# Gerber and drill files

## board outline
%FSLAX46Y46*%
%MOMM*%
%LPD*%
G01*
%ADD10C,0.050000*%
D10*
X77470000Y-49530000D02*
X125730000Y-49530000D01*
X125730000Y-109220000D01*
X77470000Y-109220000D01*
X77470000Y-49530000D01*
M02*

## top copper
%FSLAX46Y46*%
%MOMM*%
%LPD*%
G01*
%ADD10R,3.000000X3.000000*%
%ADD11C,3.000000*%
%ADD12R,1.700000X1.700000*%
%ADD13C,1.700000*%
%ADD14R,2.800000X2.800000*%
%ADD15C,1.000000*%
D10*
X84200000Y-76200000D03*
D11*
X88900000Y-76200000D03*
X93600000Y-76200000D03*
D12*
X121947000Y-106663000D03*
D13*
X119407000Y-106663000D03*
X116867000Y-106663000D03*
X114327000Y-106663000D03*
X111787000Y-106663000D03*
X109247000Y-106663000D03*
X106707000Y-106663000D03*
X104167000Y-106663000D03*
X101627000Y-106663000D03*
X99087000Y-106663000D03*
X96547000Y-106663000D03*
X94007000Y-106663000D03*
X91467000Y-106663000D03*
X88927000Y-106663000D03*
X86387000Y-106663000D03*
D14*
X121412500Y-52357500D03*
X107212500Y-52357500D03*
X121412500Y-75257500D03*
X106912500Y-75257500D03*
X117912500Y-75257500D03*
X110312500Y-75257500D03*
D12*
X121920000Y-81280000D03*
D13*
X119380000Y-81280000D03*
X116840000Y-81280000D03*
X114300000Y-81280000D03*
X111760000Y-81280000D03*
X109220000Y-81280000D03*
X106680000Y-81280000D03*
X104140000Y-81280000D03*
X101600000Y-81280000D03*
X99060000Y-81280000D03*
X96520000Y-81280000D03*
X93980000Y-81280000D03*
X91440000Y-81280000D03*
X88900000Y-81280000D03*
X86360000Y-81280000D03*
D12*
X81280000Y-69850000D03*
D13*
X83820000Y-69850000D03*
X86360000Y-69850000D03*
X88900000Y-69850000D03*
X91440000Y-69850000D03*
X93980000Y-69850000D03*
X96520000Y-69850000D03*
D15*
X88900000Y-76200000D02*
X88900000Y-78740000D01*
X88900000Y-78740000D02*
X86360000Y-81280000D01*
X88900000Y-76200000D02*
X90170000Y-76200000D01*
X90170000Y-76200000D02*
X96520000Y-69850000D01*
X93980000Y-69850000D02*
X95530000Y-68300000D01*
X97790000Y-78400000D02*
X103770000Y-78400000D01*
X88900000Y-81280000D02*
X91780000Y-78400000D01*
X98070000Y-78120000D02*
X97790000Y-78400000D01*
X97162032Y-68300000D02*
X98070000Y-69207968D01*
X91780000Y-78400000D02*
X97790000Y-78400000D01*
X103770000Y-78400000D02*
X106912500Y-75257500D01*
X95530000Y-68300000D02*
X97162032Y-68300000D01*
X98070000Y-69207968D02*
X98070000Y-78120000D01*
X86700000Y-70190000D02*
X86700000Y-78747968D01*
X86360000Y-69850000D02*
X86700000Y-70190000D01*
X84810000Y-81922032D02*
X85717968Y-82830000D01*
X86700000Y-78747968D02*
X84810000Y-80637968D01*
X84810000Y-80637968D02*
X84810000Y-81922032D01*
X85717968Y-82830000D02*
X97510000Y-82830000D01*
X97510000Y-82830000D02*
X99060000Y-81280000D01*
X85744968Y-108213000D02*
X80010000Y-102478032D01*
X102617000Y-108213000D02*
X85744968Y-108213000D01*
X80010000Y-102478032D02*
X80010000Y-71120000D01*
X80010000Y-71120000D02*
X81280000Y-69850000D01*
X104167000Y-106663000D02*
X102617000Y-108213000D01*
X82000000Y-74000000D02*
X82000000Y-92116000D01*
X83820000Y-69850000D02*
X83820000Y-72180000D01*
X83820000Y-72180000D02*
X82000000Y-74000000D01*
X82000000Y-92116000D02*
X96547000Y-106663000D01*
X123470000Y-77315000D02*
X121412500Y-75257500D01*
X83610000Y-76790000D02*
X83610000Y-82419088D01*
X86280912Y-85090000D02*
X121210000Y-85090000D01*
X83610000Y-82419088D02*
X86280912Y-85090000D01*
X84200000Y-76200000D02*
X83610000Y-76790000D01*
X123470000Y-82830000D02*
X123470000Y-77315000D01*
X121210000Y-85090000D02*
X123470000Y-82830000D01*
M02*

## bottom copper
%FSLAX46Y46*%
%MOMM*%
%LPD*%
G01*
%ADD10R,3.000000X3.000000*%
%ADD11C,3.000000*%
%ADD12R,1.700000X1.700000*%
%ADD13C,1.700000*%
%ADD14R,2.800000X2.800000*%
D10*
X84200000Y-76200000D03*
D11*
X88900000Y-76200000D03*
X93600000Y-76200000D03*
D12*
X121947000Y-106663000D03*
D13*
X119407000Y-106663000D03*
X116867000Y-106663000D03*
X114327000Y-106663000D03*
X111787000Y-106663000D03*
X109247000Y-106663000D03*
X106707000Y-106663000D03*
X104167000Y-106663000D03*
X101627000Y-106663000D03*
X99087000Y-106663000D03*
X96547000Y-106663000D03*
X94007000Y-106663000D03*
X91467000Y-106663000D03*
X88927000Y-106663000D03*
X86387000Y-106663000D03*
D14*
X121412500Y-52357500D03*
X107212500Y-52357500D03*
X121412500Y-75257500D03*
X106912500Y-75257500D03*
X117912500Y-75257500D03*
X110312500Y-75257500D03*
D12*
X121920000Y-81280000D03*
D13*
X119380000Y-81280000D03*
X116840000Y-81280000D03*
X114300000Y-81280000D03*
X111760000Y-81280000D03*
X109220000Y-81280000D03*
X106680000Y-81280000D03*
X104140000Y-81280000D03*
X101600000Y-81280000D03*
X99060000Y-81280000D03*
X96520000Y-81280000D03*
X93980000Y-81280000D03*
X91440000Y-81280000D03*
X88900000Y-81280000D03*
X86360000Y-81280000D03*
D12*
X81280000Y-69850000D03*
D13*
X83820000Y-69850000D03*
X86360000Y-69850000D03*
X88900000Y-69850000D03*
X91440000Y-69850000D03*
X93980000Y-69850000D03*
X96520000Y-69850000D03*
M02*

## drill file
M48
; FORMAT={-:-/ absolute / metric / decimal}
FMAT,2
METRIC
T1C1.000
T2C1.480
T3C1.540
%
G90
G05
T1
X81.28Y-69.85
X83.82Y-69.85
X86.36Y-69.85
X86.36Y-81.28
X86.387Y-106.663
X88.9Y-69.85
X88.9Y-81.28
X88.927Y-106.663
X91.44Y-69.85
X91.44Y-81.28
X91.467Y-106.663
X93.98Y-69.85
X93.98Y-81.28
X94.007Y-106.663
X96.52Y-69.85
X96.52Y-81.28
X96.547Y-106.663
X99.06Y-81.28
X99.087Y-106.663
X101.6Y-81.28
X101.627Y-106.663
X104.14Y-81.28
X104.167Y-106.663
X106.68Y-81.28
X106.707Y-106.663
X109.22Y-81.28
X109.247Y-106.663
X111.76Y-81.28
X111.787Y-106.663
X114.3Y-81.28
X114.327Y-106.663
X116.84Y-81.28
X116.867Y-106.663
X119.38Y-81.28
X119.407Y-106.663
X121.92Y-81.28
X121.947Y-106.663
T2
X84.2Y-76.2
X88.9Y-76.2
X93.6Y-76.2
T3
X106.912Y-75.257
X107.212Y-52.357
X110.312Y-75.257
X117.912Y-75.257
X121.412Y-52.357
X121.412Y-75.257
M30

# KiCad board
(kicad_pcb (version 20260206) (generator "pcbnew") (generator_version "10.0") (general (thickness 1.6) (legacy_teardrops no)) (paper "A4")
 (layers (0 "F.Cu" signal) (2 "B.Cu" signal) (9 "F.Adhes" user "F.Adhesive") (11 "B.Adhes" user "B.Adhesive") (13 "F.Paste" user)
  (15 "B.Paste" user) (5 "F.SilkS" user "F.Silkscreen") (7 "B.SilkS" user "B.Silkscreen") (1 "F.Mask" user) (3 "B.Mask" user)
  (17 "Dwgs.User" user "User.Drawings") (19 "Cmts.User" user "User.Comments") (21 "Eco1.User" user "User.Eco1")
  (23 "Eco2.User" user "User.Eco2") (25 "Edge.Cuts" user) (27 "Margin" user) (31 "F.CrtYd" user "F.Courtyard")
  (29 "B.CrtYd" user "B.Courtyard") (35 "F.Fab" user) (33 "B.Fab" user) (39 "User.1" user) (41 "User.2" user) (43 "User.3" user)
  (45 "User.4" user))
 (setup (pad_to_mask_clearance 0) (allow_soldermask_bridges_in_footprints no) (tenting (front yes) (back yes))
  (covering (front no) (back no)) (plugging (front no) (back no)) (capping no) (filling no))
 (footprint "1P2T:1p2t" (layer "F.Cu") (at 88.9 76.2)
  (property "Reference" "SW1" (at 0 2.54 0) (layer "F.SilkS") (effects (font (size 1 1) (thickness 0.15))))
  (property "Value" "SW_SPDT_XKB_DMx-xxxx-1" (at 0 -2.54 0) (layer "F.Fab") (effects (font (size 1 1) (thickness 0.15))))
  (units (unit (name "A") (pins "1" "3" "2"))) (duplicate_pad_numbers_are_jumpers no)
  (pad "1" thru_hole rect (at -4.7 0) (size 3 3) (drill 1.48) (layers "*.Cu" "*.Mask") (remove_unused_layers no) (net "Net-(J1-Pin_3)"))
  (pad "2" thru_hole circle (at 0 0) (size 3 3) (drill 1.48) (layers "*.Cu" "*.Mask") (remove_unused_layers no) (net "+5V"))
  (pad "3" thru_hole circle (at 4.7 0) (size 3 3) (drill 1.48) (layers "*.Cu" "*.Mask") (remove_unused_layers no)
   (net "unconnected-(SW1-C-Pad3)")))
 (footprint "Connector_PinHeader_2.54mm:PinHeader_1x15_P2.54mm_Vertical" (layer "F.Cu") (at 121.947 106.663 -90)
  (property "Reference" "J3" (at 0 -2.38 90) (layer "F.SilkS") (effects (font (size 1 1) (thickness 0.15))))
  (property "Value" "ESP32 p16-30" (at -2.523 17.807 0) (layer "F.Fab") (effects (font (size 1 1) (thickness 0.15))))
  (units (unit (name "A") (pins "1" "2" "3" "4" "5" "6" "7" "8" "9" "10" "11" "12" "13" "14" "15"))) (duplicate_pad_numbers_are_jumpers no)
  (pad "1" thru_hole rect (at 0 0 270) (size 1.7 1.7) (drill 1) (layers "*.Cu" "*.Mask") (remove_unused_layers no)
   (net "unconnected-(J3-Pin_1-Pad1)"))
  (pad "2" thru_hole circle (at 0 2.54 270) (size 1.7 1.7) (drill 1) (layers "*.Cu" "*.Mask") (remove_unused_layers no)
   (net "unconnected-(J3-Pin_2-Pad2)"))
  (pad "3" thru_hole circle (at 0 5.08 270) (size 1.7 1.7) (drill 1) (layers "*.Cu" "*.Mask") (remove_unused_layers no)
   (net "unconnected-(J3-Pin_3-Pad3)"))
  (pad "4" thru_hole circle (at 0 7.62 270) (size 1.7 1.7) (drill 1) (layers "*.Cu" "*.Mask") (remove_unused_layers no)
   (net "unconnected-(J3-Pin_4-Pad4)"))
  (pad "5" thru_hole circle (at 0 10.16 270) (size 1.7 1.7) (drill 1) (layers "*.Cu" "*.Mask") (remove_unused_layers no)
   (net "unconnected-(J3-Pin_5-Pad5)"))
  (pad "6" thru_hole circle (at 0 12.7 270) (size 1.7 1.7) (drill 1) (layers "*.Cu" "*.Mask") (remove_unused_layers no)
   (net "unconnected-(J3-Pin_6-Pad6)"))
  (pad "7" thru_hole circle (at 0 15.24 270) (size 1.7 1.7) (drill 1) (layers "*.Cu" "*.Mask") (remove_unused_layers no)
   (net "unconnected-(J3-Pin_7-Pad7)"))
  (pad "8" thru_hole circle (at 0 17.78 270) (size 1.7 1.7) (drill 1) (layers "*.Cu" "*.Mask") (remove_unused_layers no) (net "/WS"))
  (pad "9" thru_hole circle (at 0 20.32 270) (size 1.7 1.7) (drill 1) (layers "*.Cu" "*.Mask") (remove_unused_layers no)
   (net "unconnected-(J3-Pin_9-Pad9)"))
  (pad "10" thru_hole circle (at 0 22.86 270) (size 1.7 1.7) (drill 1) (layers "*.Cu" "*.Mask") (remove_unused_layers no)
   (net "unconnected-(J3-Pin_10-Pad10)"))
  (pad "11" thru_hole circle (at 0 25.4 270) (size 1.7 1.7) (drill 1) (layers "*.Cu" "*.Mask") (remove_unused_layers no) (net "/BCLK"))
  (pad "12" thru_hole circle (at 0 27.94 270) (size 1.7 1.7) (drill 1) (layers "*.Cu" "*.Mask") (remove_unused_layers no)
   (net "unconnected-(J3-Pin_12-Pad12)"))
  (pad "13" thru_hole circle (at 0 30.48 270) (size 1.7 1.7) (drill 1) (layers "*.Cu" "*.Mask") (remove_unused_layers no)
   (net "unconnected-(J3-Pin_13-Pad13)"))
  (pad "14" thru_hole circle (at 0 33.02 270) (size 1.7 1.7) (drill 1) (layers "*.Cu" "*.Mask") (remove_unused_layers no)
   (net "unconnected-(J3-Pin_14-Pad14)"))
  (pad "15" thru_hole circle (at 0 35.56 270) (size 1.7 1.7) (drill 1) (layers "*.Cu" "*.Mask") (remove_unused_layers no)
   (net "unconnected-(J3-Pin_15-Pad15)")))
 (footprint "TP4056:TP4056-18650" (layer "F.Cu") (at 123.1125 50.6575 -90)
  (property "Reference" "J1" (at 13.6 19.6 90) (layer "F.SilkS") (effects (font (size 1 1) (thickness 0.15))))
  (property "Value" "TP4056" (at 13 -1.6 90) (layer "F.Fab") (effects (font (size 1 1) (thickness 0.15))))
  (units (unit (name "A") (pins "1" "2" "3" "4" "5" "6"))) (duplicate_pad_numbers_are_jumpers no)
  (pad "1" thru_hole rect (at 1.7 1.7 270) (size 2.8 2.8) (drill 1.54) (layers "*.Cu" "*.Mask") (remove_unused_layers no)
   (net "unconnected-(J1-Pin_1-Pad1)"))
  (pad "2" thru_hole rect (at 1.7 15.9 270) (size 2.8 2.8) (drill 1.54) (layers "*.Cu" "*.Mask") (remove_unused_layers no)
   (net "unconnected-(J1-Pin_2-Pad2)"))
  (pad "3" thru_hole rect (at 24.6 1.7 270) (size 2.8 2.8) (drill 1.54) (layers "*.Cu" "*.Mask") (remove_unused_layers no)
   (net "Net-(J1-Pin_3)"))
  (pad "4" thru_hole rect (at 24.6 16.2 270) (size 2.8 2.8) (drill 1.54) (layers "*.Cu" "*.Mask") (remove_unused_layers no) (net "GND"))
  (pad "5" thru_hole rect (at 24.6 5.2 270) (size 2.8 2.8) (drill 1.54) (layers "*.Cu" "*.Mask") (remove_unused_layers no) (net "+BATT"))
  (pad "6" thru_hole rect (at 24.6 12.8 270) (size 2.8 2.8) (drill 1.54) (layers "*.Cu" "*.Mask") (remove_unused_layers no) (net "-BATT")))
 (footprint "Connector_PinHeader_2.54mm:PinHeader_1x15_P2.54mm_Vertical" (layer "F.Cu") (at 121.92 81.28 -90)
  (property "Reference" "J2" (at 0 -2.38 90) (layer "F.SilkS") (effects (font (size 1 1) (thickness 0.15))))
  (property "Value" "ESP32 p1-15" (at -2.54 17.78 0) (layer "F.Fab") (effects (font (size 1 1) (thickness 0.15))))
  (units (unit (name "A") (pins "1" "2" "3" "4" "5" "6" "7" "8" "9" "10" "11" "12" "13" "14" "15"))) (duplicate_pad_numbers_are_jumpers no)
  (pad "1" thru_hole rect (at 0 0 270) (size 1.7 1.7) (drill 1) (layers "*.Cu" "*.Mask") (remove_unused_layers no)
   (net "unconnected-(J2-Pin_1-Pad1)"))
  (pad "2" thru_hole circle (at 0 2.54 270) (size 1.7 1.7) (drill 1) (layers "*.Cu" "*.Mask") (remove_unused_layers no)
   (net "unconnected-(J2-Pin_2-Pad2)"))
  (pad "3" thru_hole circle (at 0 5.08 270) (size 1.7 1.7) (drill 1) (layers "*.Cu" "*.Mask") (remove_unused_layers no)
   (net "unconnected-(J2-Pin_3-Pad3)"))
  (pad "4" thru_hole circle (at 0 7.62 270) (size 1.7 1.7) (drill 1) (layers "*.Cu" "*.Mask") (remove_unused_layers no)
   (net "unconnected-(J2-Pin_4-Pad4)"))
  (pad "5" thru_hole circle (at 0 10.16 270) (size 1.7 1.7) (drill 1) (layers "*.Cu" "*.Mask") (remove_unused_layers no)
   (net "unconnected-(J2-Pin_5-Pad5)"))
  (pad "6" thru_hole circle (at 0 12.7 270) (size 1.7 1.7) (drill 1) (layers "*.Cu" "*.Mask") (remove_unused_layers no)
   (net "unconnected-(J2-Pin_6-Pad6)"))
  (pad "7" thru_hole circle (at 0 15.24 270) (size 1.7 1.7) (drill 1) (layers "*.Cu" "*.Mask") (remove_unused_layers no)
   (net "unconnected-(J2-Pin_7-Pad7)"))
  (pad "8" thru_hole circle (at 0 17.78 270) (size 1.7 1.7) (drill 1) (layers "*.Cu" "*.Mask") (remove_unused_layers no)
   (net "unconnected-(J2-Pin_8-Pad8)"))
  (pad "9" thru_hole circle (at 0 20.32 270) (size 1.7 1.7) (drill 1) (layers "*.Cu" "*.Mask") (remove_unused_layers no)
   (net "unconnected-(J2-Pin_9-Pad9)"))
  (pad "10" thru_hole circle (at 0 22.86 270) (size 1.7 1.7) (drill 1) (layers "*.Cu" "*.Mask") (remove_unused_layers no) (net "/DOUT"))
  (pad "11" thru_hole circle (at 0 25.4 270) (size 1.7 1.7) (drill 1) (layers "*.Cu" "*.Mask") (remove_unused_layers no)
   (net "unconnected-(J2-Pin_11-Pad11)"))
  (pad "12" thru_hole circle (at 0 27.94 270) (size 1.7 1.7) (drill 1) (layers "*.Cu" "*.Mask") (remove_unused_layers no)
   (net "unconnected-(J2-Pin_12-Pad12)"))
  (pad "13" thru_hole circle (at 0 30.48 270) (size 1.7 1.7) (drill 1) (layers "*.Cu" "*.Mask") (remove_unused_layers no)
   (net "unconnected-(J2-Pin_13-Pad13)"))
  (pad "14" thru_hole circle (at 0 33.02 270) (size 1.7 1.7) (drill 1) (layers "*.Cu" "*.Mask") (remove_unused_layers no) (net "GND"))
  (pad "15" thru_hole circle (at 0 35.56 270) (size 1.7 1.7) (drill 1) (layers "*.Cu" "*.Mask") (remove_unused_layers no) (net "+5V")))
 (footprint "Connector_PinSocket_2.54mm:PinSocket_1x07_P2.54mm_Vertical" (layer "F.Cu") (at 81.28 69.85 90)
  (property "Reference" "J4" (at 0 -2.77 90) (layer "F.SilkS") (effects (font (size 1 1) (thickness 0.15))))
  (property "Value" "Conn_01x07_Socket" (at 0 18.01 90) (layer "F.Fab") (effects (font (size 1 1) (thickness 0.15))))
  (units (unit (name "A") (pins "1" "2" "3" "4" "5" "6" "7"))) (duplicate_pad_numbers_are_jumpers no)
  (pad "1" thru_hole rect (at 0 0 90) (size 1.7 1.7) (drill 1) (layers "*.Cu" "*.Mask") (remove_unused_layers no) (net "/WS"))
  (pad "2" thru_hole circle (at 0 2.54 90) (size 1.7 1.7) (drill 1) (layers "*.Cu" "*.Mask") (remove_unused_layers no) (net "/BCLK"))
  (pad "3" thru_hole circle (at 0 5.08 90) (size 1.7 1.7) (drill 1) (layers "*.Cu" "*.Mask") (remove_unused_layers no) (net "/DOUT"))
  (pad "4" thru_hole circle (at 0 7.62 90) (size 1.7 1.7) (drill 1) (layers "*.Cu" "*.Mask") (remove_unused_layers no)
   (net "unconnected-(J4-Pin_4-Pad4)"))
  (pad "5" thru_hole circle (at 0 10.16 90) (size 1.7 1.7) (drill 1) (layers "*.Cu" "*.Mask") (remove_unused_layers no)
   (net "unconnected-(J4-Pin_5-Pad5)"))
  (pad "6" thru_hole circle (at 0 12.7 90) (size 1.7 1.7) (drill 1) (layers "*.Cu" "*.Mask") (remove_unused_layers no) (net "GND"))
  (pad "7" thru_hole circle (at 0 15.24 90) (size 1.7 1.7) (drill 1) (layers "*.Cu" "*.Mask") (remove_unused_layers no) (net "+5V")))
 (gr_rect (start 77.47 49.53) (end 125.73 109.22) (stroke (width 0.05) (type default)) (fill no) (layer "Edge.Cuts"))
 (segment (start 88.9 76.2) (end 88.9 78.74) (width 1) (layer "F.Cu") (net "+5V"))
 (segment (start 88.9 78.74) (end 86.36 81.28) (width 1) (layer "F.Cu") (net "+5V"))
 (segment (start 88.9 76.2) (end 90.17 76.2) (width 1) (layer "F.Cu") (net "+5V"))
 (segment (start 90.17 76.2) (end 96.52 69.85) (width 1) (layer "F.Cu") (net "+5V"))
 (segment (start 93.98 69.85) (end 95.53 68.3) (width 1) (layer "F.Cu") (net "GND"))
 (segment (start 97.79 78.4) (end 103.77 78.4) (width 1) (layer "F.Cu") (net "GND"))
 (segment (start 88.9 81.28) (end 91.78 78.4) (width 1) (layer "F.Cu") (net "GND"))
 (segment (start 98.07 78.12) (end 97.79 78.4) (width 1) (layer "F.Cu") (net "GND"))
 (segment (start 97.162032 68.3) (end 98.07 69.207968) (width 1) (layer "F.Cu") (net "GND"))
 (segment (start 91.78 78.4) (end 97.79 78.4) (width 1) (layer "F.Cu") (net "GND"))
 (segment (start 103.77 78.4) (end 106.9125 75.2575) (width 1) (layer "F.Cu") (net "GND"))
 (segment (start 95.53 68.3) (end 97.162032 68.3) (width 1) (layer "F.Cu") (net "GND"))
 (segment (start 98.07 69.207968) (end 98.07 78.12) (width 1) (layer "F.Cu") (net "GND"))
 (segment (start 86.7 70.19) (end 86.7 78.747968) (width 1) (layer "F.Cu") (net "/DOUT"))
 (segment (start 86.36 69.85) (end 86.7 70.19) (width 1) (layer "F.Cu") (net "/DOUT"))
 (segment (start 84.81 81.922032) (end 85.717968 82.83) (width 1) (layer "F.Cu") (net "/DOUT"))
 (segment (start 86.7 78.747968) (end 84.81 80.637968) (width 1) (layer "F.Cu") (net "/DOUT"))
 (segment (start 84.81 80.637968) (end 84.81 81.922032) (width 1) (layer "F.Cu") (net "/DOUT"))
 (segment (start 85.717968 82.83) (end 97.51 82.83) (width 1) (layer "F.Cu") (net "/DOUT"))
 (segment (start 97.51 82.83) (end 99.06 81.28) (width 1) (layer "F.Cu") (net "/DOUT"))
 (segment (start 85.744968 108.213) (end 80.01 102.478032) (width 1) (layer "F.Cu") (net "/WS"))
 (segment (start 102.617 108.213) (end 85.744968 108.213) (width 1) (layer "F.Cu") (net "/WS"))
 (segment (start 80.01 102.478032) (end 80.01 71.12) (width 1) (layer "F.Cu") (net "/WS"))
 (segment (start 80.01 71.12) (end 81.28 69.85) (width 1) (layer "F.Cu") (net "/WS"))
 (segment (start 104.167 106.663) (end 102.617 108.213) (width 1) (layer "F.Cu") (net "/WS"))
 (segment (start 82 74) (end 82 92.116) (width 1) (layer "F.Cu") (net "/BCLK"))
 (segment (start 83.82 69.85) (end 83.82 72.18) (width 1) (layer "F.Cu") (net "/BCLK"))
 (segment (start 83.82 72.18) (end 82 74) (width 1) (layer "F.Cu") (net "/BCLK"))
 (segment (start 82 92.116) (end 96.547 106.663) (width 1) (layer "F.Cu") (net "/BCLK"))
 (segment (start 123.47 77.315) (end 121.4125 75.2575) (width 1) (layer "F.Cu") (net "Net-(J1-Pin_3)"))
 (segment (start 83.61 76.79) (end 83.61 82.419088) (width 1) (layer "F.Cu") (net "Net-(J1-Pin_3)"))
 (segment (start 86.280912 85.09) (end 121.21 85.09) (width 1) (layer "F.Cu") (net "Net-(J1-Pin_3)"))
 (segment (start 83.61 82.419088) (end 86.280912 85.09) (width 1) (layer "F.Cu") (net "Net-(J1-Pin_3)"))
 (segment (start 84.2 76.2) (end 83.61 76.79) (width 1) (layer "F.Cu") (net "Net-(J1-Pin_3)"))
 (segment (start 123.47 82.83) (end 123.47 77.315) (width 1) (layer "F.Cu") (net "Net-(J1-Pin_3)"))
 (segment (start 121.21 85.09) (end 123.47 82.83) (width 1) (layer "F.Cu") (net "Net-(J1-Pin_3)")))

